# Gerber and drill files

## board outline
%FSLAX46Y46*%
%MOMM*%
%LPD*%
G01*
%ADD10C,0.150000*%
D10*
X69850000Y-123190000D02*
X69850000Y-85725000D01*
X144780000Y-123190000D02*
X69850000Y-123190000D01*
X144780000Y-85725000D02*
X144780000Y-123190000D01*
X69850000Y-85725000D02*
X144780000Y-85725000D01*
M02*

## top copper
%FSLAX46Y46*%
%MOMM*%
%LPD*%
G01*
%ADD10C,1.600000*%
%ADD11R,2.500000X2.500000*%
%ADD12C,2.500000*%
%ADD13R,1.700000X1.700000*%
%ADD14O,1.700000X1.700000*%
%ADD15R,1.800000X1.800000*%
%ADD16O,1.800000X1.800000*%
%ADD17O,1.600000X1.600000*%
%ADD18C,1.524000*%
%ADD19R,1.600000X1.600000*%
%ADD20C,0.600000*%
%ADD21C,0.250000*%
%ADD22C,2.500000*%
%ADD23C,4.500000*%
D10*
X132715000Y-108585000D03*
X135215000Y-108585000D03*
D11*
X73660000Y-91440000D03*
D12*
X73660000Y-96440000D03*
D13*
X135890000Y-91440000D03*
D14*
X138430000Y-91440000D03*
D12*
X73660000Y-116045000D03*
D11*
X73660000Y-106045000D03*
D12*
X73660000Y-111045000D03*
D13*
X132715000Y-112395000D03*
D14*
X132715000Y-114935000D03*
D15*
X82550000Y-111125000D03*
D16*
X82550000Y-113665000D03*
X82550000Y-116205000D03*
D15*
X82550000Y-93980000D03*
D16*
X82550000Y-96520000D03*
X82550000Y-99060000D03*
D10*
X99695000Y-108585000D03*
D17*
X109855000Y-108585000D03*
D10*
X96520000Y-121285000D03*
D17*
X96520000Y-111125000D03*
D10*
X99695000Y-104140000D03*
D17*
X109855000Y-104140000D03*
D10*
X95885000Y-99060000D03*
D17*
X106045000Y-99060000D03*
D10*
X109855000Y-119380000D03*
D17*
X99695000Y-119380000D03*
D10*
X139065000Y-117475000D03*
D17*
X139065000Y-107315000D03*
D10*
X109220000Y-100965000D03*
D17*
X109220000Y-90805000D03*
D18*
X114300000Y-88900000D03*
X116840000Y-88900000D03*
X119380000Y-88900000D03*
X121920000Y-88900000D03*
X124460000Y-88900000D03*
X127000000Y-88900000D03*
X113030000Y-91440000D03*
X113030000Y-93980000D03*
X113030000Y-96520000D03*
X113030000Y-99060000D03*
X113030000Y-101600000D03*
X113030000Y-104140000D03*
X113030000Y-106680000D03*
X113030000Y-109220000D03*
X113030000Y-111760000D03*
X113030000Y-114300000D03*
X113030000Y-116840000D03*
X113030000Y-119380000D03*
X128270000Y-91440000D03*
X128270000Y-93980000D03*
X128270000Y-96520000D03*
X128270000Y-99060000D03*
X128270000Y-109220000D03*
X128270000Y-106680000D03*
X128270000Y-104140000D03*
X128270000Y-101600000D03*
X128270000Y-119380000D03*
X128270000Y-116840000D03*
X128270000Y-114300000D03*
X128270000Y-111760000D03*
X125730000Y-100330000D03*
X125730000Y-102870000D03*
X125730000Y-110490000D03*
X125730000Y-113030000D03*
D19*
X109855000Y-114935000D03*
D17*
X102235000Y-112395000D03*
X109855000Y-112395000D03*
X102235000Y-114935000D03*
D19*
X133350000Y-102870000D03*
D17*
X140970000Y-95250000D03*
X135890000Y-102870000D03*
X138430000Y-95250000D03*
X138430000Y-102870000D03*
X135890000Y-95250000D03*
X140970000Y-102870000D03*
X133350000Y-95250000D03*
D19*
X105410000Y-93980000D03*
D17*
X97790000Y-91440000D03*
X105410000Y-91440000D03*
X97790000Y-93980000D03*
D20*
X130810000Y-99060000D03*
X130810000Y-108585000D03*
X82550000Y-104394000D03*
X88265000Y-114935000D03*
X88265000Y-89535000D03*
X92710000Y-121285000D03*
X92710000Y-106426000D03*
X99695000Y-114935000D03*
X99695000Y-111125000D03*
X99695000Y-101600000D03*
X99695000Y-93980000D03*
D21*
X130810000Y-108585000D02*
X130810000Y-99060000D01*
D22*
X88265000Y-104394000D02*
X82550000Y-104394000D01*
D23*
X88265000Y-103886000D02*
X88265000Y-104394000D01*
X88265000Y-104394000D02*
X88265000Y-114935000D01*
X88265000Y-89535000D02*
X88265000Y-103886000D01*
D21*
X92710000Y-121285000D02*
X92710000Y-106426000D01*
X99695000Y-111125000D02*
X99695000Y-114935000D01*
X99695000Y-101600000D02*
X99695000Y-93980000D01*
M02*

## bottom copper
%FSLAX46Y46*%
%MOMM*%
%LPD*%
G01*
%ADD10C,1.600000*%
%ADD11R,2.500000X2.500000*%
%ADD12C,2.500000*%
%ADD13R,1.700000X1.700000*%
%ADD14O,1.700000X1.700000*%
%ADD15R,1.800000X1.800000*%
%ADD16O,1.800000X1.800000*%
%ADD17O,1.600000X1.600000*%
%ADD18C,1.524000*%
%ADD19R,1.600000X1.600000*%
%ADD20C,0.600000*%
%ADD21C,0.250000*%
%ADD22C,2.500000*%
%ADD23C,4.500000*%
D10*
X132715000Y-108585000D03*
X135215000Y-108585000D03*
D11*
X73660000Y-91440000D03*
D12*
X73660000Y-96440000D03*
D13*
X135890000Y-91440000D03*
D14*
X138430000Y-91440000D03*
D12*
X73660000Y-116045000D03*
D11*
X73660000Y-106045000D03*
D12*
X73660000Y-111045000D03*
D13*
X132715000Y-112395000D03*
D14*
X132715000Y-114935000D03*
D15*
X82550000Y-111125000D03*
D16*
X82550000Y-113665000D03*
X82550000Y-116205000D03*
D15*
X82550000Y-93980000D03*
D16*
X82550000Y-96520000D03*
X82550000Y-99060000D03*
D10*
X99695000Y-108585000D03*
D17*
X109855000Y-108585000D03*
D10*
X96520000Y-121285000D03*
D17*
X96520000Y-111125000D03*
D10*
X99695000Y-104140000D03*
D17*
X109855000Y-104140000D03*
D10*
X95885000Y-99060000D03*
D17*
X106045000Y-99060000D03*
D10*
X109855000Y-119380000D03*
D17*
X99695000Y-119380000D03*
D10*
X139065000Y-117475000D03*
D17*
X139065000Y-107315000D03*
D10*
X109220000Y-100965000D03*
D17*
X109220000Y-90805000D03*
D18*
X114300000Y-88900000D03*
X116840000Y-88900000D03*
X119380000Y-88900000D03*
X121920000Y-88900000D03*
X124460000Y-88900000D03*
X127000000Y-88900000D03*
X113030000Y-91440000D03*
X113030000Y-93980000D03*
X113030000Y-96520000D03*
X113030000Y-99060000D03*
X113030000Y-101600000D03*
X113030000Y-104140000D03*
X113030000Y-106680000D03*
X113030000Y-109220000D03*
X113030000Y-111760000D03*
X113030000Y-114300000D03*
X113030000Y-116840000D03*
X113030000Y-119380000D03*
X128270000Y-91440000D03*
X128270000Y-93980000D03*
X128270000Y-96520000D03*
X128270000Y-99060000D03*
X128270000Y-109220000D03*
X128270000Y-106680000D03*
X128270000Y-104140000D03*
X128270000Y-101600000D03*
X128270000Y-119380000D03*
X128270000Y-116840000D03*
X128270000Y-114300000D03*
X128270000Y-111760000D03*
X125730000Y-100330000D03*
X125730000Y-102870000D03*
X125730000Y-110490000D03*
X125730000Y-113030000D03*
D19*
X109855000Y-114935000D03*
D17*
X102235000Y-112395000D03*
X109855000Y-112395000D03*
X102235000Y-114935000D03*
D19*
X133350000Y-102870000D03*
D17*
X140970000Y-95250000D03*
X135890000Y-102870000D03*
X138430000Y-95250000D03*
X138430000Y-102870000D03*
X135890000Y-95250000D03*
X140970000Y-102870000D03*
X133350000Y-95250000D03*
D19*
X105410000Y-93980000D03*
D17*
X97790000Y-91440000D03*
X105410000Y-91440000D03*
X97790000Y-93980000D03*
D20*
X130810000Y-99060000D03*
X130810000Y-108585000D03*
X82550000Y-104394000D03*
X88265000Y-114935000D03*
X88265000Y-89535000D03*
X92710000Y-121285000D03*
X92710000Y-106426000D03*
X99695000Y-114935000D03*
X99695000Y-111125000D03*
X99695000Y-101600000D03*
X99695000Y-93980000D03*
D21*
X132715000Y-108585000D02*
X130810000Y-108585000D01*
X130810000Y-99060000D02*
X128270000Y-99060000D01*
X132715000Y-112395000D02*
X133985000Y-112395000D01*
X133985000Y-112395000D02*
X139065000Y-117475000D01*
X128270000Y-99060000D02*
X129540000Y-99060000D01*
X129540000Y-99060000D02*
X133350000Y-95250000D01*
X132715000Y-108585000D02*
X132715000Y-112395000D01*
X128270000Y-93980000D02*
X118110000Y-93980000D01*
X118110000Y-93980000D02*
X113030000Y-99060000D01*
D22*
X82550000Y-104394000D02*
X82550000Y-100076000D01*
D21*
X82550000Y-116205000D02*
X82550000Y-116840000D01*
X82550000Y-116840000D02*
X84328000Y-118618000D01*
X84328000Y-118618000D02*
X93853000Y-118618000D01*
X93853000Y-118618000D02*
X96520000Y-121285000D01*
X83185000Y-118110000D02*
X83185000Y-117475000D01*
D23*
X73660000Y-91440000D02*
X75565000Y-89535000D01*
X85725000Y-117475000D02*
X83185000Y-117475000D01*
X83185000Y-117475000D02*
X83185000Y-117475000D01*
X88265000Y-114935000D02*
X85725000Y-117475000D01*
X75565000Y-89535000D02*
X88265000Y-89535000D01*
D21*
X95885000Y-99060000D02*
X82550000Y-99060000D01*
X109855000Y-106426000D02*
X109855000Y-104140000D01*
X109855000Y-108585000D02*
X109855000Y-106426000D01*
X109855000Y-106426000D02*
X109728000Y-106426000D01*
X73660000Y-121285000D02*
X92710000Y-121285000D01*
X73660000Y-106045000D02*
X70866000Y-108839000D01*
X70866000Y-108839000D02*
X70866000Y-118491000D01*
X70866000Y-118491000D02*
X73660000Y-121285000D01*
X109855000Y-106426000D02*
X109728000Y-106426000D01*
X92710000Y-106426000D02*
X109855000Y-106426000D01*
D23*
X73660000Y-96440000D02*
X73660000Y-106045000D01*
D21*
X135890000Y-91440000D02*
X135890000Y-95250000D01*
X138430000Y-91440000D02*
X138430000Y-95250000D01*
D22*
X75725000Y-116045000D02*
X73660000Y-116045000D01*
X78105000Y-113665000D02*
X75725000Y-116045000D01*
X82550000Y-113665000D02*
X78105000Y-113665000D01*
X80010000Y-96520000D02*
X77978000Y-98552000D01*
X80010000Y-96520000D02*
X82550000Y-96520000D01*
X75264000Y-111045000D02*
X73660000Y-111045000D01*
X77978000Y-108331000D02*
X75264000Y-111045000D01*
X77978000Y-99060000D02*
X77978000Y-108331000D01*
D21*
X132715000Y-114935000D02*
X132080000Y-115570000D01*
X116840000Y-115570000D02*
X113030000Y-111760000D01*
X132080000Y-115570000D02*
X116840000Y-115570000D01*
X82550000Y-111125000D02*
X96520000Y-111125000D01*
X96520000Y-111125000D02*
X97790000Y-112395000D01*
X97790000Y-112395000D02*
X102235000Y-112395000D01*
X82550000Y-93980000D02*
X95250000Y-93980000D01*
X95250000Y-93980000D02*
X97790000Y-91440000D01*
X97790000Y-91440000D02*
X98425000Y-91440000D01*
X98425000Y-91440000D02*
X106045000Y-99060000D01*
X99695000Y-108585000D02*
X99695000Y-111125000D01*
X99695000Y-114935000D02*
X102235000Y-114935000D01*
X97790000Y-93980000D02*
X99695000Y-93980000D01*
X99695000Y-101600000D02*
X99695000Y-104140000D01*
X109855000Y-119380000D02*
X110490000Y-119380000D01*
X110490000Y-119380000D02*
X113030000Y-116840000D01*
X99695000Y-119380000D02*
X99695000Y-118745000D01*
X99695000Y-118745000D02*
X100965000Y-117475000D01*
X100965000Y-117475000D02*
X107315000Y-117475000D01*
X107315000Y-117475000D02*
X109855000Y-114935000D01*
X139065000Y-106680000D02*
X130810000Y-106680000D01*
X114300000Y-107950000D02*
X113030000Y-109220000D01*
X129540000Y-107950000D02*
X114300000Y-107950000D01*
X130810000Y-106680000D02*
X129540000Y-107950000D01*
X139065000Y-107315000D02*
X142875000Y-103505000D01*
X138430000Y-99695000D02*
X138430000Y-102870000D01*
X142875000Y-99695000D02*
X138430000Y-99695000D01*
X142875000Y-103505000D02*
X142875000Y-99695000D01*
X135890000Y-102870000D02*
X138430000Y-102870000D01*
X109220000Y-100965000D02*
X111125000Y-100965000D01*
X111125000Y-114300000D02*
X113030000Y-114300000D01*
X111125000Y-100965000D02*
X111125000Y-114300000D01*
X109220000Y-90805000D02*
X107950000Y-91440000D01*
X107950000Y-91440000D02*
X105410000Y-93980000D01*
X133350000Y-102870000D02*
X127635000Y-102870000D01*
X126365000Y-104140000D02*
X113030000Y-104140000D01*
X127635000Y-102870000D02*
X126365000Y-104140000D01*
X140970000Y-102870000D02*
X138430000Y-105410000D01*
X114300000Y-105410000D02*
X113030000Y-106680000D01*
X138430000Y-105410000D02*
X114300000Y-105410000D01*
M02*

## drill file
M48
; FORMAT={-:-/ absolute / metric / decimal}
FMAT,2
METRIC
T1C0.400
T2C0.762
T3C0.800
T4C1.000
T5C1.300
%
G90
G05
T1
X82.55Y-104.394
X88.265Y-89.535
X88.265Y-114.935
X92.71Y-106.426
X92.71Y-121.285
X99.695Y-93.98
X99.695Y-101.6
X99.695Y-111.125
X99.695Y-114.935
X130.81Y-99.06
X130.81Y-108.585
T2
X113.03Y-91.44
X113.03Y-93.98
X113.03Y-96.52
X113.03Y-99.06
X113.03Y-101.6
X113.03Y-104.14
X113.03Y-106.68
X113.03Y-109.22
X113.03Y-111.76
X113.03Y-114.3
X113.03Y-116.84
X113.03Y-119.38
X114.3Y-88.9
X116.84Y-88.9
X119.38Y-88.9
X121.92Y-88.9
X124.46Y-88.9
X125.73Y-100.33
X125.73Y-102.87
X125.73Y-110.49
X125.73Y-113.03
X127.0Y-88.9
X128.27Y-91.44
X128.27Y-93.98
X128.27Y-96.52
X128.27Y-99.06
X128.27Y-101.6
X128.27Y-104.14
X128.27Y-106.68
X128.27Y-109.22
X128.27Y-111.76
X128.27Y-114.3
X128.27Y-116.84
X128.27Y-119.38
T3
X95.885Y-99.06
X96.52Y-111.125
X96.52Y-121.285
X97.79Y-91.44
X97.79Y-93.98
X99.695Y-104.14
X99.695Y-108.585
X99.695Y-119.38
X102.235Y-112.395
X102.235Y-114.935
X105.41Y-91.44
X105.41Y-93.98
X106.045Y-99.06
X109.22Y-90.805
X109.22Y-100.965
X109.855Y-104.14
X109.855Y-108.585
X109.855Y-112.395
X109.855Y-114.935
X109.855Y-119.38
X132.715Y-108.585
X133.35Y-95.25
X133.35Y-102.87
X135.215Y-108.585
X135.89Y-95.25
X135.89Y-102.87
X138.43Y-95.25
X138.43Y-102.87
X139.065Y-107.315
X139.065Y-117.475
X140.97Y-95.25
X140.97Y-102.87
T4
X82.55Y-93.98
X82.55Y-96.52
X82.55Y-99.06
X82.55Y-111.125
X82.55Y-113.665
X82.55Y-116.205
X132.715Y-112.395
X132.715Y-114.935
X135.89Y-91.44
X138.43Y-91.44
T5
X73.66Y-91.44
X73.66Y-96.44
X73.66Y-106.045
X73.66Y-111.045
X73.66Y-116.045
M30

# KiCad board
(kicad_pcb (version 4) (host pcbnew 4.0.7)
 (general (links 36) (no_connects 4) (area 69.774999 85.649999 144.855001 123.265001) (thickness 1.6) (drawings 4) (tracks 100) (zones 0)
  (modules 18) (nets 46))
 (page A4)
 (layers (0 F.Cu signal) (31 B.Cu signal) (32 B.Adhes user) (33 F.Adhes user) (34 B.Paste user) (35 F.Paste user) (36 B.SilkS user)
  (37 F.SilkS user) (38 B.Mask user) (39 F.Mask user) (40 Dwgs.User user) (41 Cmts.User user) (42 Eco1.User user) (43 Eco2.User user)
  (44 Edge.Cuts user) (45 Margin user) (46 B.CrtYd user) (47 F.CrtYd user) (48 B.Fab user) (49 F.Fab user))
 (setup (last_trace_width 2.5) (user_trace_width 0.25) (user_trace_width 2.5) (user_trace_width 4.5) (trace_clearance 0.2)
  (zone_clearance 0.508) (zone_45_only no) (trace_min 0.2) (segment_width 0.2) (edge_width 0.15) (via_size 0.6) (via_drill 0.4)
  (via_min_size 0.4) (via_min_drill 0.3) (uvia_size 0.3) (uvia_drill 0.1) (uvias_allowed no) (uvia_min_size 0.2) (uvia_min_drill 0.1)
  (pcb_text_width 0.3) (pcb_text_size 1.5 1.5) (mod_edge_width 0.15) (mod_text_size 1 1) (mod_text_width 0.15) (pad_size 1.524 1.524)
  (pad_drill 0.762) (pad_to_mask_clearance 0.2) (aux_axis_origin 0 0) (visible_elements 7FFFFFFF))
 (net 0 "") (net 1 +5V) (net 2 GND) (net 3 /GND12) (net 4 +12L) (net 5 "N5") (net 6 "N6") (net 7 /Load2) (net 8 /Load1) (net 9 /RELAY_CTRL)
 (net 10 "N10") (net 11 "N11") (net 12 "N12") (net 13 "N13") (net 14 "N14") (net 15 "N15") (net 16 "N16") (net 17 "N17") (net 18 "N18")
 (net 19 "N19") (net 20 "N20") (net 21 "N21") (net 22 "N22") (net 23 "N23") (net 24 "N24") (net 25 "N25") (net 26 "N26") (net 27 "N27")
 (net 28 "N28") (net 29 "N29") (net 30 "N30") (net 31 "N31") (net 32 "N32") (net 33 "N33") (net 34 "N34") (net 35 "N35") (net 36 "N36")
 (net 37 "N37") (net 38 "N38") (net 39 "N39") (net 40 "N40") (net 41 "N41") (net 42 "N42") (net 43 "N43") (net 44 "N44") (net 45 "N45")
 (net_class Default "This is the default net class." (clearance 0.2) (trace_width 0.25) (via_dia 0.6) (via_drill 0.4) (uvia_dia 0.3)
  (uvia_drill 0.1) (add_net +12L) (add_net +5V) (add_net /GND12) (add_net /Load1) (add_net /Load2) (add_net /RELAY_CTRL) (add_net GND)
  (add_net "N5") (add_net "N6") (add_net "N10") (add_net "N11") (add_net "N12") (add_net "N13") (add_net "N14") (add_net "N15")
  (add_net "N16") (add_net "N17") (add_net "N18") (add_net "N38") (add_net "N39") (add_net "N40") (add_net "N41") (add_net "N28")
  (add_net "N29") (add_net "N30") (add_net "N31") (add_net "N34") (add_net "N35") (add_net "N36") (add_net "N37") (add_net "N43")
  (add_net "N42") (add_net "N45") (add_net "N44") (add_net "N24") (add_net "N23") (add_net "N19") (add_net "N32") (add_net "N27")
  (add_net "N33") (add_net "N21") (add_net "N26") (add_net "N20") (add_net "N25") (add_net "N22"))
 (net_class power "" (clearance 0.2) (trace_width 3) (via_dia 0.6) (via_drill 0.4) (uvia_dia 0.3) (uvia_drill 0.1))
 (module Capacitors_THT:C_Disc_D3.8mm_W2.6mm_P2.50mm (layer F.Cu) (at 132.715 108.585)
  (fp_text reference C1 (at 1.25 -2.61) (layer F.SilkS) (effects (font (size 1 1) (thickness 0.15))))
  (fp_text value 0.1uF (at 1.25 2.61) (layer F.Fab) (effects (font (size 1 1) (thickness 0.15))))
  (pad 1 thru_hole circle (at 0 0) (size 1.6 1.6) (drill 0.8) (layers *.Cu *.Mask) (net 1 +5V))
  (pad 2 thru_hole circle (at 2.5 0) (size 1.6 1.6) (drill 0.8) (layers *.Cu *.Mask) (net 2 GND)))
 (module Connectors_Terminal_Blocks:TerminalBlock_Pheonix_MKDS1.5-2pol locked (layer F.Cu) (at 73.66 91.44 270)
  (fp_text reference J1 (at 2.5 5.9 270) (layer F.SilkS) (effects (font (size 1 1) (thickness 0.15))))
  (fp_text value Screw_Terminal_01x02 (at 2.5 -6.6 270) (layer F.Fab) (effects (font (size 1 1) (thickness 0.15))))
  (pad 1 thru_hole rect (at 0 0 270) (size 2.5 2.5) (drill 1.3) (layers *.Cu *.Mask) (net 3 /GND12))
  (pad 2 thru_hole circle (at 5 0 270) (size 2.5 2.5) (drill 1.3) (layers *.Cu *.Mask) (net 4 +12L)))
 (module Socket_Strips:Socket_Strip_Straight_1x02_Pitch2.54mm (layer F.Cu) (at 135.89 91.44 90)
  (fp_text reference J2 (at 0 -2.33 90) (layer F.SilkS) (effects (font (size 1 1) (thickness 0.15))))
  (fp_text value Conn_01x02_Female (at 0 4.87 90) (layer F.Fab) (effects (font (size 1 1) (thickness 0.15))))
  (pad 1 thru_hole rect (at 0 0 90) (size 1.7 1.7) (drill 1) (layers *.Cu *.Mask) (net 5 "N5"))
  (pad 2 thru_hole oval (at 0 2.54 90) (size 1.7 1.7) (drill 1) (layers *.Cu *.Mask) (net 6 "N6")))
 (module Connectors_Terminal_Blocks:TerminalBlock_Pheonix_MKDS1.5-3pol (layer F.Cu) (at 73.66 106.045 270)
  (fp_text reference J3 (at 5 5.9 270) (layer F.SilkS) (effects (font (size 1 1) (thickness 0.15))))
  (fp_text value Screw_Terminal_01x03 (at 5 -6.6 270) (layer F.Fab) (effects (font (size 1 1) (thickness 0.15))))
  (pad 3 thru_hole circle (at 10 0 270) (size 2.5 2.5) (drill 1.3) (layers *.Cu *.Mask) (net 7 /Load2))
  (pad 1 thru_hole rect (at 0 0 270) (size 2.5 2.5) (drill 1.3) (layers *.Cu *.Mask) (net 4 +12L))
  (pad 2 thru_hole circle (at 5 0 270) (size 2.5 2.5) (drill 1.3) (layers *.Cu *.Mask) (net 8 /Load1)))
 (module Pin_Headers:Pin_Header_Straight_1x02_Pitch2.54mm (layer F.Cu) (at 132.715 112.395)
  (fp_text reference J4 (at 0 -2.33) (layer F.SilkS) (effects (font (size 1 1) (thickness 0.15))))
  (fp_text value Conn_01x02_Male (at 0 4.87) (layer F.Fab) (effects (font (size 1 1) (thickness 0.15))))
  (pad 1 thru_hole rect (at 0 0) (size 1.7 1.7) (drill 1) (layers *.Cu *.Mask) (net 1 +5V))
  (pad 2 thru_hole oval (at 0 2.54) (size 1.7 1.7) (drill 1) (layers *.Cu *.Mask) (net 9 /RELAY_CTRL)))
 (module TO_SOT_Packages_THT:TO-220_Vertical (layer F.Cu) (at 82.55 111.125 270)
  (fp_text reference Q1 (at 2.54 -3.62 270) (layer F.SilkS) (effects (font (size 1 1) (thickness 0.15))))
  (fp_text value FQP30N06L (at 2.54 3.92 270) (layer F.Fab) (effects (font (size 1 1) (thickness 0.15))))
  (pad 1 thru_hole rect (at 0 0 270) (size 1.8 1.8) (drill 1) (layers *.Cu *.Mask) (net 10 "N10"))
  (pad 2 thru_hole oval (at 2.54 0 270) (size 1.8 1.8) (drill 1) (layers *.Cu *.Mask) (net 7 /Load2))
  (pad 3 thru_hole oval (at 5.08 0 270) (size 1.8 1.8) (drill 1) (layers *.Cu *.Mask) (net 3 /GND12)))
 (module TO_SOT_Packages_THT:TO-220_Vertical (layer F.Cu) (at 82.55 93.98 270)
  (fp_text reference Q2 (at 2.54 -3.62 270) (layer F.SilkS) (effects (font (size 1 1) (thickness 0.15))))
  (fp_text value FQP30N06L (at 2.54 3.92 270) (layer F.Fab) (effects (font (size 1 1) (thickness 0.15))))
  (pad 1 thru_hole rect (at 0 0 270) (size 1.8 1.8) (drill 1) (layers *.Cu *.Mask) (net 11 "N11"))
  (pad 2 thru_hole oval (at 2.54 0 270) (size 1.8 1.8) (drill 1) (layers *.Cu *.Mask) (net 8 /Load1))
  (pad 3 thru_hole oval (at 5.08 0 270) (size 1.8 1.8) (drill 1) (layers *.Cu *.Mask) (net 3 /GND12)))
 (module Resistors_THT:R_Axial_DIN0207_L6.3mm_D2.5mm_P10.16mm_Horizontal (layer F.Cu) (at 99.695 108.585)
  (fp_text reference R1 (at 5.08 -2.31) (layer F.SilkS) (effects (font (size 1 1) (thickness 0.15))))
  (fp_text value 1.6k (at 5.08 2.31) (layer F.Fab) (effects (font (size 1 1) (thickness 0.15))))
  (pad 1 thru_hole circle (at 0 0) (size 1.6 1.6) (drill 0.8) (layers *.Cu *.Mask) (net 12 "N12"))
  (pad 2 thru_hole oval (at 10.16 0) (size 1.6 1.6) (drill 0.8) (layers *.Cu *.Mask) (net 4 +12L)))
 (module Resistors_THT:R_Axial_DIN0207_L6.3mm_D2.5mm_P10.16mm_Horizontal (layer F.Cu) (at 96.52 121.285 90)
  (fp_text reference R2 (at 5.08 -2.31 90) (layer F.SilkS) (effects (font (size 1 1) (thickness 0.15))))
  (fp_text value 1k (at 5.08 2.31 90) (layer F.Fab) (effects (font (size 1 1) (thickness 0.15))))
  (pad 1 thru_hole circle (at 0 0 90) (size 1.6 1.6) (drill 0.8) (layers *.Cu *.Mask) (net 3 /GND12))
  (pad 2 thru_hole oval (at 10.16 0 90) (size 1.6 1.6) (drill 0.8) (layers *.Cu *.Mask) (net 10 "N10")))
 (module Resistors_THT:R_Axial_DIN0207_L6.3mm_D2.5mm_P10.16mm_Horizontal (layer F.Cu) (at 99.695 104.14)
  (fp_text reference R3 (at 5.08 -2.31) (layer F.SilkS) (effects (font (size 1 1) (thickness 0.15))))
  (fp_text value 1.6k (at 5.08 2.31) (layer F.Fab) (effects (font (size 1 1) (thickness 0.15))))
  (pad 1 thru_hole circle (at 0 0) (size 1.6 1.6) (drill 0.8) (layers *.Cu *.Mask) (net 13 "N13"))
  (pad 2 thru_hole oval (at 10.16 0) (size 1.6 1.6) (drill 0.8) (layers *.Cu *.Mask) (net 4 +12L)))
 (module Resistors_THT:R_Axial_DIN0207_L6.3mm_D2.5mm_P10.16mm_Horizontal (layer F.Cu) (at 95.885 99.06)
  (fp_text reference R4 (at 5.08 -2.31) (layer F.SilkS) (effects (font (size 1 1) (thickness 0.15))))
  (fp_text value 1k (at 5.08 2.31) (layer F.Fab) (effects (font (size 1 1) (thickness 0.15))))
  (pad 1 thru_hole circle (at 0 0) (size 1.6 1.6) (drill 0.8) (layers *.Cu *.Mask) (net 3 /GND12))
  (pad 2 thru_hole oval (at 10.16 0) (size 1.6 1.6) (drill 0.8) (layers *.Cu *.Mask) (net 11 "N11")))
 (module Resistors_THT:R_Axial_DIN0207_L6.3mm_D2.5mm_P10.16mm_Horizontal (layer F.Cu) (at 109.855 119.38 180)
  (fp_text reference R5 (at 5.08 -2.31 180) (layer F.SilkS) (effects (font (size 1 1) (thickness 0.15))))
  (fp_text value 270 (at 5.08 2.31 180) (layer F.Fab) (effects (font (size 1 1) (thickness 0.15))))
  (pad 1 thru_hole circle (at 0 0 180) (size 1.6 1.6) (drill 0.8) (layers *.Cu *.Mask) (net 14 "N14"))
  (pad 2 thru_hole oval (at 10.16 0 180) (size 1.6 1.6) (drill 0.8) (layers *.Cu *.Mask) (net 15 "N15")))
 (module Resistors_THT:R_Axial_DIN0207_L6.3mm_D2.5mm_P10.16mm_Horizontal (layer F.Cu) (at 139.065 117.475 90)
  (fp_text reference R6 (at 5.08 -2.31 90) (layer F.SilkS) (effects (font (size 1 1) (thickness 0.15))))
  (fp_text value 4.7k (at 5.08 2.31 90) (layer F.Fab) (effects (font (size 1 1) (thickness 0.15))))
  (pad 1 thru_hole circle (at 0 0 90) (size 1.6 1.6) (drill 0.8) (layers *.Cu *.Mask) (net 1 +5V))
  (pad 2 thru_hole oval (at 10.16 0 90) (size 1.6 1.6) (drill 0.8) (layers *.Cu *.Mask) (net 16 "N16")))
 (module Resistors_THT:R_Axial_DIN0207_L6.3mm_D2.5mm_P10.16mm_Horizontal (layer F.Cu) (at 109.22 100.965 90)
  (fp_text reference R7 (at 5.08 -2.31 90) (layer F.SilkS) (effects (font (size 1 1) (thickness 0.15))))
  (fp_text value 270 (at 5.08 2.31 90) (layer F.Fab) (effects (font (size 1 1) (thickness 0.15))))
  (pad 1 thru_hole circle (at 0 0 90) (size 1.6 1.6) (drill 0.8) (layers *.Cu *.Mask) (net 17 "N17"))
  (pad 2 thru_hole oval (at 10.16 0 90) (size 1.6 1.6) (drill 0.8) (layers *.Cu *.Mask) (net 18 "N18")))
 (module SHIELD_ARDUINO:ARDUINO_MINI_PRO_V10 (layer F.Cu) (at 120.65 104.14)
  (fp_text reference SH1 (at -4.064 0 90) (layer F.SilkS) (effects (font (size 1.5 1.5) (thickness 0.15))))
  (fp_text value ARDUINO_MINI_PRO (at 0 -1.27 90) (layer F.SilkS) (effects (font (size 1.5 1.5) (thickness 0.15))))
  (pad GRN thru_hole circle (at -6.35 -15.24) (size 1.524 1.524) (drill 0.762) (layers *.Cu *.Mask F.SilkS) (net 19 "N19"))
  (pad TX/1 thru_hole circle (at -3.81 -15.24) (size 1.524 1.524) (drill 0.762) (layers *.Cu *.Mask F.SilkS) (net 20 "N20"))
  (pad RX/1 thru_hole circle (at -1.27 -15.24) (size 1.524 1.524) (drill 0.762) (layers *.Cu *.Mask F.SilkS) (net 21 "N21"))
  (pad VCC1 thru_hole circle (at 1.27 -15.24) (size 1.524 1.524) (drill 0.762) (layers *.Cu *.Mask F.SilkS) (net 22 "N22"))
  (pad GND1 thru_hole circle (at 3.81 -15.24) (size 1.524 1.524) (drill 0.762) (layers *.Cu *.Mask F.SilkS) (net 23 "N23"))
  (pad BLK thru_hole circle (at 6.35 -15.24) (size 1.524 1.524) (drill 0.762) (layers *.Cu *.Mask F.SilkS) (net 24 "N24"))
  (pad TX/2 thru_hole circle (at -7.62 -12.7) (size 1.524 1.524) (drill 0.762) (layers *.Cu *.Mask F.SilkS) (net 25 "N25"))
  (pad RX/2 thru_hole circle (at -7.62 -10.16) (size 1.524 1.524) (drill 0.762) (layers *.Cu *.Mask F.SilkS) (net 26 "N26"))
  (pad RST1 thru_hole circle (at -7.62 -7.62) (size 1.524 1.524) (drill 0.762) (layers *.Cu *.Mask F.SilkS) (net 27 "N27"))
  (pad GND2 thru_hole circle (at -7.62 -5.08) (size 1.524 1.524) (drill 0.762) (layers *.Cu *.Mask F.SilkS) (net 2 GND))
  (pad 2 thru_hole circle (at -7.62 -2.54) (size 1.524 1.524) (drill 0.762) (layers *.Cu *.Mask F.SilkS) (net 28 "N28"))
  (pad 3 thru_hole circle (at -7.62 0) (size 1.524 1.524) (drill 0.762) (layers *.Cu *.Mask F.SilkS) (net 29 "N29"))
  (pad 4 thru_hole circle (at -7.62 2.54) (size 1.524 1.524) (drill 0.762) (layers *.Cu *.Mask F.SilkS) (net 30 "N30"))
  (pad 5 thru_hole circle (at -7.62 5.08) (size 1.524 1.524) (drill 0.762) (layers *.Cu *.Mask F.SilkS) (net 16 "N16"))
  (pad 6 thru_hole circle (at -7.62 7.62) (size 1.524 1.524) (drill 0.762) (layers *.Cu *.Mask F.SilkS) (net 9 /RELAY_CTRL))
  (pad 7 thru_hole circle (at -7.62 10.16) (size 1.524 1.524) (drill 0.762) (layers *.Cu *.Mask F.SilkS) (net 17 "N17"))
  (pad 8 thru_hole circle (at -7.62 12.7) (size 1.524 1.524) (drill 0.762) (layers *.Cu *.Mask F.SilkS) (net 14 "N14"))
  (pad 9 thru_hole circle (at -7.62 15.24) (size 1.524 1.524) (drill 0.762) (layers *.Cu *.Mask F.SilkS) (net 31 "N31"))
  (pad RAW thru_hole circle (at 7.62 -12.7) (size 1.524 1.524) (drill 0.762) (layers *.Cu *.Mask F.SilkS) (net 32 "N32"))
  (pad GND3 thru_hole circle (at 7.62 -10.16) (size 1.524 1.524) (drill 0.762) (layers *.Cu *.Mask F.SilkS) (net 2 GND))
  (pad RST2 thru_hole circle (at 7.62 -7.62) (size 1.524 1.524) (drill 0.762) (layers *.Cu *.Mask F.SilkS) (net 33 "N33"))
  (pad VCC2 thru_hole circle (at 7.62 -5.08) (size 1.524 1.524) (drill 0.762) (layers *.Cu *.Mask F.SilkS) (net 1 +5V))
  (pad A0 thru_hole circle (at 7.62 5.08) (size 1.524 1.524) (drill 0.762) (layers *.Cu *.Mask F.SilkS) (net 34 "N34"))
  (pad A1 thru_hole circle (at 7.62 2.54) (size 1.524 1.524) (drill 0.762) (layers *.Cu *.Mask F.SilkS) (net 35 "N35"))
  (pad A2 thru_hole circle (at 7.62 0) (size 1.524 1.524) (drill 0.762) (layers *.Cu *.Mask F.SilkS) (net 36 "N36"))
  (pad A3 thru_hole circle (at 7.62 -2.54) (size 1.524 1.524) (drill 0.762) (layers *.Cu *.Mask F.SilkS) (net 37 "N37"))
  (pad 10 thru_hole circle (at 7.62 15.24) (size 1.524 1.524) (drill 0.762) (layers *.Cu *.Mask F.SilkS) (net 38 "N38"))
  (pad 11 thru_hole circle (at 7.62 12.7) (size 1.524 1.524) (drill 0.762) (layers *.Cu *.Mask F.SilkS) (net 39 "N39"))
  (pad 12 thru_hole circle (at 7.62 10.16) (size 1.524 1.524) (drill 0.762) (layers *.Cu *.Mask F.SilkS) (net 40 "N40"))
  (pad 13 thru_hole circle (at 7.62 7.62) (size 1.524 1.524) (drill 0.762) (layers *.Cu *.Mask F.SilkS) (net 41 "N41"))
  (pad A5 thru_hole circle (at 5.08 -3.81) (size 1.524 1.524) (drill 0.762) (layers *.Cu *.Mask F.SilkS) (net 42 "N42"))
  (pad A4 thru_hole circle (at 5.08 -1.27) (size 1.524 1.524) (drill 0.762) (layers *.Cu *.Mask F.SilkS) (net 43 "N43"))
  (pad A7 thru_hole circle (at 5.08 6.35) (size 1.524 1.524) (drill 0.762) (layers *.Cu *.Mask F.SilkS) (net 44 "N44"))
  (pad A6 thru_hole circle (at 5.08 8.89) (size 1.524 1.524) (drill 0.762) (layers *.Cu *.Mask F.SilkS) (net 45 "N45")))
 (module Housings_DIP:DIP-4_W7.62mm (layer F.Cu) (at 109.855 114.935 180)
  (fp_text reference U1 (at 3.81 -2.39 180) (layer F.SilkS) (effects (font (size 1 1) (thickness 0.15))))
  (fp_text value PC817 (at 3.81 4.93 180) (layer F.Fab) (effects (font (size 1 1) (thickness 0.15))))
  (pad 1 thru_hole rect (at 0 0 180) (size 1.6 1.6) (drill 0.8) (layers *.Cu *.Mask) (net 15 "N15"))
  (pad 3 thru_hole oval (at 7.62 2.54 180) (size 1.6 1.6) (drill 0.8) (layers *.Cu *.Mask) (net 10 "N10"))
  (pad 2 thru_hole oval (at 0 2.54 180) (size 1.6 1.6) (drill 0.8) (layers *.Cu *.Mask) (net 2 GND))
  (pad 4 thru_hole oval (at 7.62 0 180) (size 1.6 1.6) (drill 0.8) (layers *.Cu *.Mask) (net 12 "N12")))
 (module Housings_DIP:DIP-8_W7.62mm (layer F.Cu) (at 133.35 102.87 90)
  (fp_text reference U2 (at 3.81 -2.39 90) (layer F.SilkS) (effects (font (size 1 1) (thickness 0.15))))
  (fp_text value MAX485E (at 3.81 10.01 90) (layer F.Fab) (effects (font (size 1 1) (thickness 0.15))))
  (pad 1 thru_hole rect (at 0 0 90) (size 1.6 1.6) (drill 0.8) (layers *.Cu *.Mask) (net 29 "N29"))
  (pad 5 thru_hole oval (at 7.62 7.62 90) (size 1.6 1.6) (drill 0.8) (layers *.Cu *.Mask) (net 2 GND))
  (pad 2 thru_hole oval (at 0 2.54 90) (size 1.6 1.6) (drill 0.8) (layers *.Cu *.Mask) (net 16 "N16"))
  (pad 6 thru_hole oval (at 7.62 5.08 90) (size 1.6 1.6) (drill 0.8) (layers *.Cu *.Mask) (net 6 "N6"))
  (pad 3 thru_hole oval (at 0 5.08 90) (size 1.6 1.6) (drill 0.8) (layers *.Cu *.Mask) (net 16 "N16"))
  (pad 7 thru_hole oval (at 7.62 2.54 90) (size 1.6 1.6) (drill 0.8) (layers *.Cu *.Mask) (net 5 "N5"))
  (pad 4 thru_hole oval (at 0 7.62 90) (size 1.6 1.6) (drill 0.8) (layers *.Cu *.Mask) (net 30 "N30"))
  (pad 8 thru_hole oval (at 7.62 0 90) (size 1.6 1.6) (drill 0.8) (layers *.Cu *.Mask) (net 1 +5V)))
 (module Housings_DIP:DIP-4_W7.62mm (layer F.Cu) (at 105.41 93.98 180)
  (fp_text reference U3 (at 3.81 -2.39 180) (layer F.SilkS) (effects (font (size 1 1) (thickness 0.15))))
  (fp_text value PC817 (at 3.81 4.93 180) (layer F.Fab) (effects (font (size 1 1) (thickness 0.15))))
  (pad 1 thru_hole rect (at 0 0 180) (size 1.6 1.6) (drill 0.8) (layers *.Cu *.Mask) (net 18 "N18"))
  (pad 3 thru_hole oval (at 7.62 2.54 180) (size 1.6 1.6) (drill 0.8) (layers *.Cu *.Mask) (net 11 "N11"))
  (pad 2 thru_hole oval (at 0 2.54 180) (size 1.6 1.6) (drill 0.8) (layers *.Cu *.Mask) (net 2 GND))
  (pad 4 thru_hole oval (at 7.62 0 180) (size 1.6 1.6) (drill 0.8) (layers *.Cu *.Mask) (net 13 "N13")))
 (gr_line (start 69.85 123.19) (end 69.85 85.725) (angle 90) (layer Edge.Cuts) (width 0.15))
 (gr_line (start 144.78 123.19) (end 69.85 123.19) (angle 90) (layer Edge.Cuts) (width 0.15))
 (gr_line (start 144.78 85.725) (end 144.78 123.19) (angle 90) (layer Edge.Cuts) (width 0.15))
 (gr_line (start 69.85 85.725) (end 144.78 85.725) (angle 90) (layer Edge.Cuts) (width 0.15))
 (segment (start 132.715 108.585) (end 130.81 108.585) (width 0.25) (layer B.Cu) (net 1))
 (segment (start 130.81 99.06) (end 128.27 99.06) (width 0.25) (layer B.Cu) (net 1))
 (via (at 130.81 99.06) (size 0.6) (drill 0.4) (layers F.Cu B.Cu) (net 1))
 (segment (start 130.81 108.585) (end 130.81 99.06) (width 0.25) (layer F.Cu) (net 1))
 (via (at 130.81 108.585) (size 0.6) (drill 0.4) (layers F.Cu B.Cu) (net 1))
 (segment (start 132.715 112.395) (end 133.985 112.395) (width 0.25) (layer B.Cu) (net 1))
 (segment (start 133.985 112.395) (end 139.065 117.475) (width 0.25) (layer B.Cu) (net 1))
 (segment (start 128.27 99.06) (end 129.54 99.06) (width 0.25) (layer B.Cu) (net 1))
 (segment (start 129.54 99.06) (end 133.35 95.25) (width 0.25) (layer B.Cu) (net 1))
 (segment (start 132.715 108.585) (end 132.715 112.395) (width 0.25) (layer B.Cu) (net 1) (status 10))
 (segment (start 128.27 93.98) (end 118.11 93.98) (width 0.25) (layer B.Cu) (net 2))
 (segment (start 118.11 93.98) (end 113.03 99.06) (width 0.25) (layer B.Cu) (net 2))
 (segment (start 88.265 104.394) (end 82.55 104.394) (width 2.5) (layer F.Cu) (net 3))
 (segment (start 82.55 104.394) (end 82.55 100.076) (width 2.5) (layer B.Cu) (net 3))
 (via (at 82.55 104.394) (size 0.6) (drill 0.4) (layers F.Cu B.Cu) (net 3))
 (segment (start 88.265 103.886) (end 88.265 104.394) (width 4.5) (layer F.Cu) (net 3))
 (segment (start 88.265 104.394) (end 88.265 114.935) (width 4.5) (layer F.Cu) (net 3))
 (segment (start 82.55 116.205) (end 82.55 116.84) (width 0.25) (layer B.Cu) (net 3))
 (segment (start 82.55 116.84) (end 84.328 118.618) (width 0.25) (layer B.Cu) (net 3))
 (segment (start 84.328 118.618) (end 93.853 118.618) (width 0.25) (layer B.Cu) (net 3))
 (segment (start 93.853 118.618) (end 96.52 121.285) (width 0.25) (layer B.Cu) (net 3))
 (segment (start 83.185 118.11) (end 83.185 117.475) (width 0.25) (layer B.Cu) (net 3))
 (segment (start 73.66 91.44) (end 75.565 89.535) (width 4.5) (layer B.Cu) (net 3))
 (segment (start 85.725 117.475) (end 83.185 117.475) (width 4.5) (layer B.Cu) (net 3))
 (segment (start 83.185 117.475) (end 83.185 117.475) (width 4.5) (layer B.Cu) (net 3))
 (segment (start 88.265 114.935) (end 85.725 117.475) (width 4.5) (layer B.Cu) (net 3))
 (via (at 88.265 114.935) (size 0.6) (drill 0.4) (layers F.Cu B.Cu) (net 3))
 (segment (start 88.265 89.535) (end 88.265 103.886) (width 4.5) (layer F.Cu) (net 3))
 (via (at 88.265 89.535) (size 0.6) (drill 0.4) (layers F.Cu B.Cu) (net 3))
 (segment (start 75.565 89.535) (end 88.265 89.535) (width 4.5) (layer B.Cu) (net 3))
 (segment (start 95.885 99.06) (end 82.55 99.06) (width 0.25) (layer B.Cu) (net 3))
 (segment (start 109.855 106.426) (end 109.855 104.14) (width 0.25) (layer B.Cu) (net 4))
 (segment (start 109.855 108.585) (end 109.855 106.426) (width 0.25) (layer B.Cu) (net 4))
 (segment (start 109.855 106.426) (end 109.728 106.426) (width 0.25) (layer B.Cu) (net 4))
 (segment (start 92.71 121.285) (end 92.71 106.426) (width 0.25) (layer F.Cu) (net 4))
 (segment (start 73.66 121.285) (end 92.71 121.285) (width 0.25) (layer B.Cu) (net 4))
 (via (at 92.71 121.285) (size 0.6) (drill 0.4) (layers F.Cu B.Cu) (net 4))
 (segment (start 73.66 106.045) (end 70.866 108.839) (width 0.25) (layer B.Cu) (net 4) (status 10))
 (segment (start 70.866 108.839) (end 70.866 118.491) (width 0.25) (layer B.Cu) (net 4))
 (segment (start 70.866 118.491) (end 73.66 121.285) (width 0.25) (layer B.Cu) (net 4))
 (segment (start 109.855 106.426) (end 109.728 106.426) (width 0.25) (layer B.Cu) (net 4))
 (segment (start 92.71 106.426) (end 109.855 106.426) (width 0.25) (layer B.Cu) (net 4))
 (via (at 92.71 106.426) (size 0.6) (drill 0.4) (layers F.Cu B.Cu) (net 4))
 (segment (start 73.66 96.44) (end 73.66 106.045) (width 4.5) (layer B.Cu) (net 4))
 (segment (start 135.89 91.44) (end 135.89 95.25) (width 0.25) (layer B.Cu) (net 5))
 (segment (start 138.43 91.44) (end 138.43 95.25) (width 0.25) (layer B.Cu) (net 6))
 (segment (start 75.725 116.045) (end 73.66 116.045) (width 2.5) (layer B.Cu) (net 7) (status 20))
 (segment (start 78.105 113.665) (end 75.725 116.045) (width 2.5) (layer B.Cu) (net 7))
 (segment (start 82.55 113.665) (end 78.105 113.665) (width 2.5) (layer B.Cu) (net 7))
 (segment (start 80.01 96.52) (end 77.978 98.552) (width 2.5) (layer B.Cu) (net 8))
 (segment (start 80.01 96.52) (end 82.55 96.52) (width 2.5) (layer B.Cu) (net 8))
 (segment (start 75.264 111.045) (end 73.66 111.045) (width 2.5) (layer B.Cu) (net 8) (status 20))
 (segment (start 77.978 108.331) (end 75.264 111.045) (width 2.5) (layer B.Cu) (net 8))
 (segment (start 77.978 99.06) (end 77.978 108.331) (width 2.5) (layer B.Cu) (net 8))
 (segment (start 132.715 114.935) (end 132.08 115.57) (width 0.25) (layer B.Cu) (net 9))
 (segment (start 116.84 115.57) (end 113.03 111.76) (width 0.25) (layer B.Cu) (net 9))
 (segment (start 132.08 115.57) (end 116.84 115.57) (width 0.25) (layer B.Cu) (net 9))
 (segment (start 82.55 111.125) (end 96.52 111.125) (width 0.25) (layer B.Cu) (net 10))
 (segment (start 96.52 111.125) (end 97.79 112.395) (width 0.25) (layer B.Cu) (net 10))
 (segment (start 97.79 112.395) (end 102.235 112.395) (width 0.25) (layer B.Cu) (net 10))
 (segment (start 82.55 93.98) (end 95.25 93.98) (width 0.25) (layer B.Cu) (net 11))
 (segment (start 95.25 93.98) (end 97.79 91.44) (width 0.25) (layer B.Cu) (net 11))
 (segment (start 97.79 91.44) (end 98.425 91.44) (width 0.25) (layer B.Cu) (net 11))
 (segment (start 98.425 91.44) (end 106.045 99.06) (width 0.25) (layer B.Cu) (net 11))
 (segment (start 99.695 108.585) (end 99.695 111.125) (width 0.25) (layer B.Cu) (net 12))
 (segment (start 99.695 114.935) (end 102.235 114.935) (width 0.25) (layer B.Cu) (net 12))
 (via (at 99.695 114.935) (size 0.6) (drill 0.4) (layers F.Cu B.Cu) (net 12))
 (segment (start 99.695 111.125) (end 99.695 114.935) (width 0.25) (layer F.Cu) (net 12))
 (via (at 99.695 111.125) (size 0.6) (drill 0.4) (layers F.Cu B.Cu) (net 12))
 (segment (start 97.79 93.98) (end 99.695 93.98) (width 0.25) (layer B.Cu) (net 13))
 (segment (start 99.695 101.6) (end 99.695 104.14) (width 0.25) (layer B.Cu) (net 13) (status 10))
 (via (at 99.695 101.6) (size 0.6) (drill 0.4) (layers F.Cu B.Cu) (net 13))
 (segment (start 99.695 101.6) (end 99.695 93.98) (width 0.25) (layer F.Cu) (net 13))
 (via (at 99.695 93.98) (size 0.6) (drill 0.4) (layers F.Cu B.Cu) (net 13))
 (segment (start 109.855 119.38) (end 110.49 119.38) (width 0.25) (layer B.Cu) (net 14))
 (segment (start 110.49 119.38) (end 113.03 116.84) (width 0.25) (layer B.Cu) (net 14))
 (segment (start 99.695 119.38) (end 99.695 118.745) (width 0.25) (layer B.Cu) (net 15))
 (segment (start 99.695 118.745) (end 100.965 117.475) (width 0.25) (layer B.Cu) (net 15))
 (segment (start 100.965 117.475) (end 107.315 117.475) (width 0.25) (layer B.Cu) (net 15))
 (segment (start 107.315 117.475) (end 109.855 114.935) (width 0.25) (layer B.Cu) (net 15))
 (segment (start 139.065 106.68) (end 130.81 106.68) (width 0.25) (layer B.Cu) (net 16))
 (segment (start 114.3 107.95) (end 113.03 109.22) (width 0.25) (layer B.Cu) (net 16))
 (segment (start 129.54 107.95) (end 114.3 107.95) (width 0.25) (layer B.Cu) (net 16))
 (segment (start 130.81 106.68) (end 129.54 107.95) (width 0.25) (layer B.Cu) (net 16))
 (segment (start 139.065 107.315) (end 142.875 103.505) (width 0.25) (layer B.Cu) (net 16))
 (segment (start 138.43 99.695) (end 138.43 102.87) (width 0.25) (layer B.Cu) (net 16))
 (segment (start 142.875 99.695) (end 138.43 99.695) (width 0.25) (layer B.Cu) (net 16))
 (segment (start 142.875 103.505) (end 142.875 99.695) (width 0.25) (layer B.Cu) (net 16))
 (segment (start 135.89 102.87) (end 138.43 102.87) (width 0.25) (layer B.Cu) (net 16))
 (segment (start 109.22 100.965) (end 111.125 100.965) (width 0.25) (layer B.Cu) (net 17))
 (segment (start 111.125 114.3) (end 113.03 114.3) (width 0.25) (layer B.Cu) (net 17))
 (segment (start 111.125 100.965) (end 111.125 114.3) (width 0.25) (layer B.Cu) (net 17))
 (segment (start 109.22 90.805) (end 107.95 91.44) (width 0.25) (layer B.Cu) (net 18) (status 10))
 (segment (start 107.95 91.44) (end 105.41 93.98) (width 0.25) (layer B.Cu) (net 18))
 (segment (start 133.35 102.87) (end 127.635 102.87) (width 0.25) (layer B.Cu) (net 29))
 (segment (start 126.365 104.14) (end 113.03 104.14) (width 0.25) (layer B.Cu) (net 29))
 (segment (start 127.635 102.87) (end 126.365 104.14) (width 0.25) (layer B.Cu) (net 29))
 (segment (start 140.97 102.87) (end 138.43 105.41) (width 0.25) (layer B.Cu) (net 30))
 (segment (start 114.3 105.41) (end 113.03 106.68) (width 0.25) (layer B.Cu) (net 30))
 (segment (start 138.43 105.41) (end 114.3 105.41) (width 0.25) (layer B.Cu) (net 30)))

